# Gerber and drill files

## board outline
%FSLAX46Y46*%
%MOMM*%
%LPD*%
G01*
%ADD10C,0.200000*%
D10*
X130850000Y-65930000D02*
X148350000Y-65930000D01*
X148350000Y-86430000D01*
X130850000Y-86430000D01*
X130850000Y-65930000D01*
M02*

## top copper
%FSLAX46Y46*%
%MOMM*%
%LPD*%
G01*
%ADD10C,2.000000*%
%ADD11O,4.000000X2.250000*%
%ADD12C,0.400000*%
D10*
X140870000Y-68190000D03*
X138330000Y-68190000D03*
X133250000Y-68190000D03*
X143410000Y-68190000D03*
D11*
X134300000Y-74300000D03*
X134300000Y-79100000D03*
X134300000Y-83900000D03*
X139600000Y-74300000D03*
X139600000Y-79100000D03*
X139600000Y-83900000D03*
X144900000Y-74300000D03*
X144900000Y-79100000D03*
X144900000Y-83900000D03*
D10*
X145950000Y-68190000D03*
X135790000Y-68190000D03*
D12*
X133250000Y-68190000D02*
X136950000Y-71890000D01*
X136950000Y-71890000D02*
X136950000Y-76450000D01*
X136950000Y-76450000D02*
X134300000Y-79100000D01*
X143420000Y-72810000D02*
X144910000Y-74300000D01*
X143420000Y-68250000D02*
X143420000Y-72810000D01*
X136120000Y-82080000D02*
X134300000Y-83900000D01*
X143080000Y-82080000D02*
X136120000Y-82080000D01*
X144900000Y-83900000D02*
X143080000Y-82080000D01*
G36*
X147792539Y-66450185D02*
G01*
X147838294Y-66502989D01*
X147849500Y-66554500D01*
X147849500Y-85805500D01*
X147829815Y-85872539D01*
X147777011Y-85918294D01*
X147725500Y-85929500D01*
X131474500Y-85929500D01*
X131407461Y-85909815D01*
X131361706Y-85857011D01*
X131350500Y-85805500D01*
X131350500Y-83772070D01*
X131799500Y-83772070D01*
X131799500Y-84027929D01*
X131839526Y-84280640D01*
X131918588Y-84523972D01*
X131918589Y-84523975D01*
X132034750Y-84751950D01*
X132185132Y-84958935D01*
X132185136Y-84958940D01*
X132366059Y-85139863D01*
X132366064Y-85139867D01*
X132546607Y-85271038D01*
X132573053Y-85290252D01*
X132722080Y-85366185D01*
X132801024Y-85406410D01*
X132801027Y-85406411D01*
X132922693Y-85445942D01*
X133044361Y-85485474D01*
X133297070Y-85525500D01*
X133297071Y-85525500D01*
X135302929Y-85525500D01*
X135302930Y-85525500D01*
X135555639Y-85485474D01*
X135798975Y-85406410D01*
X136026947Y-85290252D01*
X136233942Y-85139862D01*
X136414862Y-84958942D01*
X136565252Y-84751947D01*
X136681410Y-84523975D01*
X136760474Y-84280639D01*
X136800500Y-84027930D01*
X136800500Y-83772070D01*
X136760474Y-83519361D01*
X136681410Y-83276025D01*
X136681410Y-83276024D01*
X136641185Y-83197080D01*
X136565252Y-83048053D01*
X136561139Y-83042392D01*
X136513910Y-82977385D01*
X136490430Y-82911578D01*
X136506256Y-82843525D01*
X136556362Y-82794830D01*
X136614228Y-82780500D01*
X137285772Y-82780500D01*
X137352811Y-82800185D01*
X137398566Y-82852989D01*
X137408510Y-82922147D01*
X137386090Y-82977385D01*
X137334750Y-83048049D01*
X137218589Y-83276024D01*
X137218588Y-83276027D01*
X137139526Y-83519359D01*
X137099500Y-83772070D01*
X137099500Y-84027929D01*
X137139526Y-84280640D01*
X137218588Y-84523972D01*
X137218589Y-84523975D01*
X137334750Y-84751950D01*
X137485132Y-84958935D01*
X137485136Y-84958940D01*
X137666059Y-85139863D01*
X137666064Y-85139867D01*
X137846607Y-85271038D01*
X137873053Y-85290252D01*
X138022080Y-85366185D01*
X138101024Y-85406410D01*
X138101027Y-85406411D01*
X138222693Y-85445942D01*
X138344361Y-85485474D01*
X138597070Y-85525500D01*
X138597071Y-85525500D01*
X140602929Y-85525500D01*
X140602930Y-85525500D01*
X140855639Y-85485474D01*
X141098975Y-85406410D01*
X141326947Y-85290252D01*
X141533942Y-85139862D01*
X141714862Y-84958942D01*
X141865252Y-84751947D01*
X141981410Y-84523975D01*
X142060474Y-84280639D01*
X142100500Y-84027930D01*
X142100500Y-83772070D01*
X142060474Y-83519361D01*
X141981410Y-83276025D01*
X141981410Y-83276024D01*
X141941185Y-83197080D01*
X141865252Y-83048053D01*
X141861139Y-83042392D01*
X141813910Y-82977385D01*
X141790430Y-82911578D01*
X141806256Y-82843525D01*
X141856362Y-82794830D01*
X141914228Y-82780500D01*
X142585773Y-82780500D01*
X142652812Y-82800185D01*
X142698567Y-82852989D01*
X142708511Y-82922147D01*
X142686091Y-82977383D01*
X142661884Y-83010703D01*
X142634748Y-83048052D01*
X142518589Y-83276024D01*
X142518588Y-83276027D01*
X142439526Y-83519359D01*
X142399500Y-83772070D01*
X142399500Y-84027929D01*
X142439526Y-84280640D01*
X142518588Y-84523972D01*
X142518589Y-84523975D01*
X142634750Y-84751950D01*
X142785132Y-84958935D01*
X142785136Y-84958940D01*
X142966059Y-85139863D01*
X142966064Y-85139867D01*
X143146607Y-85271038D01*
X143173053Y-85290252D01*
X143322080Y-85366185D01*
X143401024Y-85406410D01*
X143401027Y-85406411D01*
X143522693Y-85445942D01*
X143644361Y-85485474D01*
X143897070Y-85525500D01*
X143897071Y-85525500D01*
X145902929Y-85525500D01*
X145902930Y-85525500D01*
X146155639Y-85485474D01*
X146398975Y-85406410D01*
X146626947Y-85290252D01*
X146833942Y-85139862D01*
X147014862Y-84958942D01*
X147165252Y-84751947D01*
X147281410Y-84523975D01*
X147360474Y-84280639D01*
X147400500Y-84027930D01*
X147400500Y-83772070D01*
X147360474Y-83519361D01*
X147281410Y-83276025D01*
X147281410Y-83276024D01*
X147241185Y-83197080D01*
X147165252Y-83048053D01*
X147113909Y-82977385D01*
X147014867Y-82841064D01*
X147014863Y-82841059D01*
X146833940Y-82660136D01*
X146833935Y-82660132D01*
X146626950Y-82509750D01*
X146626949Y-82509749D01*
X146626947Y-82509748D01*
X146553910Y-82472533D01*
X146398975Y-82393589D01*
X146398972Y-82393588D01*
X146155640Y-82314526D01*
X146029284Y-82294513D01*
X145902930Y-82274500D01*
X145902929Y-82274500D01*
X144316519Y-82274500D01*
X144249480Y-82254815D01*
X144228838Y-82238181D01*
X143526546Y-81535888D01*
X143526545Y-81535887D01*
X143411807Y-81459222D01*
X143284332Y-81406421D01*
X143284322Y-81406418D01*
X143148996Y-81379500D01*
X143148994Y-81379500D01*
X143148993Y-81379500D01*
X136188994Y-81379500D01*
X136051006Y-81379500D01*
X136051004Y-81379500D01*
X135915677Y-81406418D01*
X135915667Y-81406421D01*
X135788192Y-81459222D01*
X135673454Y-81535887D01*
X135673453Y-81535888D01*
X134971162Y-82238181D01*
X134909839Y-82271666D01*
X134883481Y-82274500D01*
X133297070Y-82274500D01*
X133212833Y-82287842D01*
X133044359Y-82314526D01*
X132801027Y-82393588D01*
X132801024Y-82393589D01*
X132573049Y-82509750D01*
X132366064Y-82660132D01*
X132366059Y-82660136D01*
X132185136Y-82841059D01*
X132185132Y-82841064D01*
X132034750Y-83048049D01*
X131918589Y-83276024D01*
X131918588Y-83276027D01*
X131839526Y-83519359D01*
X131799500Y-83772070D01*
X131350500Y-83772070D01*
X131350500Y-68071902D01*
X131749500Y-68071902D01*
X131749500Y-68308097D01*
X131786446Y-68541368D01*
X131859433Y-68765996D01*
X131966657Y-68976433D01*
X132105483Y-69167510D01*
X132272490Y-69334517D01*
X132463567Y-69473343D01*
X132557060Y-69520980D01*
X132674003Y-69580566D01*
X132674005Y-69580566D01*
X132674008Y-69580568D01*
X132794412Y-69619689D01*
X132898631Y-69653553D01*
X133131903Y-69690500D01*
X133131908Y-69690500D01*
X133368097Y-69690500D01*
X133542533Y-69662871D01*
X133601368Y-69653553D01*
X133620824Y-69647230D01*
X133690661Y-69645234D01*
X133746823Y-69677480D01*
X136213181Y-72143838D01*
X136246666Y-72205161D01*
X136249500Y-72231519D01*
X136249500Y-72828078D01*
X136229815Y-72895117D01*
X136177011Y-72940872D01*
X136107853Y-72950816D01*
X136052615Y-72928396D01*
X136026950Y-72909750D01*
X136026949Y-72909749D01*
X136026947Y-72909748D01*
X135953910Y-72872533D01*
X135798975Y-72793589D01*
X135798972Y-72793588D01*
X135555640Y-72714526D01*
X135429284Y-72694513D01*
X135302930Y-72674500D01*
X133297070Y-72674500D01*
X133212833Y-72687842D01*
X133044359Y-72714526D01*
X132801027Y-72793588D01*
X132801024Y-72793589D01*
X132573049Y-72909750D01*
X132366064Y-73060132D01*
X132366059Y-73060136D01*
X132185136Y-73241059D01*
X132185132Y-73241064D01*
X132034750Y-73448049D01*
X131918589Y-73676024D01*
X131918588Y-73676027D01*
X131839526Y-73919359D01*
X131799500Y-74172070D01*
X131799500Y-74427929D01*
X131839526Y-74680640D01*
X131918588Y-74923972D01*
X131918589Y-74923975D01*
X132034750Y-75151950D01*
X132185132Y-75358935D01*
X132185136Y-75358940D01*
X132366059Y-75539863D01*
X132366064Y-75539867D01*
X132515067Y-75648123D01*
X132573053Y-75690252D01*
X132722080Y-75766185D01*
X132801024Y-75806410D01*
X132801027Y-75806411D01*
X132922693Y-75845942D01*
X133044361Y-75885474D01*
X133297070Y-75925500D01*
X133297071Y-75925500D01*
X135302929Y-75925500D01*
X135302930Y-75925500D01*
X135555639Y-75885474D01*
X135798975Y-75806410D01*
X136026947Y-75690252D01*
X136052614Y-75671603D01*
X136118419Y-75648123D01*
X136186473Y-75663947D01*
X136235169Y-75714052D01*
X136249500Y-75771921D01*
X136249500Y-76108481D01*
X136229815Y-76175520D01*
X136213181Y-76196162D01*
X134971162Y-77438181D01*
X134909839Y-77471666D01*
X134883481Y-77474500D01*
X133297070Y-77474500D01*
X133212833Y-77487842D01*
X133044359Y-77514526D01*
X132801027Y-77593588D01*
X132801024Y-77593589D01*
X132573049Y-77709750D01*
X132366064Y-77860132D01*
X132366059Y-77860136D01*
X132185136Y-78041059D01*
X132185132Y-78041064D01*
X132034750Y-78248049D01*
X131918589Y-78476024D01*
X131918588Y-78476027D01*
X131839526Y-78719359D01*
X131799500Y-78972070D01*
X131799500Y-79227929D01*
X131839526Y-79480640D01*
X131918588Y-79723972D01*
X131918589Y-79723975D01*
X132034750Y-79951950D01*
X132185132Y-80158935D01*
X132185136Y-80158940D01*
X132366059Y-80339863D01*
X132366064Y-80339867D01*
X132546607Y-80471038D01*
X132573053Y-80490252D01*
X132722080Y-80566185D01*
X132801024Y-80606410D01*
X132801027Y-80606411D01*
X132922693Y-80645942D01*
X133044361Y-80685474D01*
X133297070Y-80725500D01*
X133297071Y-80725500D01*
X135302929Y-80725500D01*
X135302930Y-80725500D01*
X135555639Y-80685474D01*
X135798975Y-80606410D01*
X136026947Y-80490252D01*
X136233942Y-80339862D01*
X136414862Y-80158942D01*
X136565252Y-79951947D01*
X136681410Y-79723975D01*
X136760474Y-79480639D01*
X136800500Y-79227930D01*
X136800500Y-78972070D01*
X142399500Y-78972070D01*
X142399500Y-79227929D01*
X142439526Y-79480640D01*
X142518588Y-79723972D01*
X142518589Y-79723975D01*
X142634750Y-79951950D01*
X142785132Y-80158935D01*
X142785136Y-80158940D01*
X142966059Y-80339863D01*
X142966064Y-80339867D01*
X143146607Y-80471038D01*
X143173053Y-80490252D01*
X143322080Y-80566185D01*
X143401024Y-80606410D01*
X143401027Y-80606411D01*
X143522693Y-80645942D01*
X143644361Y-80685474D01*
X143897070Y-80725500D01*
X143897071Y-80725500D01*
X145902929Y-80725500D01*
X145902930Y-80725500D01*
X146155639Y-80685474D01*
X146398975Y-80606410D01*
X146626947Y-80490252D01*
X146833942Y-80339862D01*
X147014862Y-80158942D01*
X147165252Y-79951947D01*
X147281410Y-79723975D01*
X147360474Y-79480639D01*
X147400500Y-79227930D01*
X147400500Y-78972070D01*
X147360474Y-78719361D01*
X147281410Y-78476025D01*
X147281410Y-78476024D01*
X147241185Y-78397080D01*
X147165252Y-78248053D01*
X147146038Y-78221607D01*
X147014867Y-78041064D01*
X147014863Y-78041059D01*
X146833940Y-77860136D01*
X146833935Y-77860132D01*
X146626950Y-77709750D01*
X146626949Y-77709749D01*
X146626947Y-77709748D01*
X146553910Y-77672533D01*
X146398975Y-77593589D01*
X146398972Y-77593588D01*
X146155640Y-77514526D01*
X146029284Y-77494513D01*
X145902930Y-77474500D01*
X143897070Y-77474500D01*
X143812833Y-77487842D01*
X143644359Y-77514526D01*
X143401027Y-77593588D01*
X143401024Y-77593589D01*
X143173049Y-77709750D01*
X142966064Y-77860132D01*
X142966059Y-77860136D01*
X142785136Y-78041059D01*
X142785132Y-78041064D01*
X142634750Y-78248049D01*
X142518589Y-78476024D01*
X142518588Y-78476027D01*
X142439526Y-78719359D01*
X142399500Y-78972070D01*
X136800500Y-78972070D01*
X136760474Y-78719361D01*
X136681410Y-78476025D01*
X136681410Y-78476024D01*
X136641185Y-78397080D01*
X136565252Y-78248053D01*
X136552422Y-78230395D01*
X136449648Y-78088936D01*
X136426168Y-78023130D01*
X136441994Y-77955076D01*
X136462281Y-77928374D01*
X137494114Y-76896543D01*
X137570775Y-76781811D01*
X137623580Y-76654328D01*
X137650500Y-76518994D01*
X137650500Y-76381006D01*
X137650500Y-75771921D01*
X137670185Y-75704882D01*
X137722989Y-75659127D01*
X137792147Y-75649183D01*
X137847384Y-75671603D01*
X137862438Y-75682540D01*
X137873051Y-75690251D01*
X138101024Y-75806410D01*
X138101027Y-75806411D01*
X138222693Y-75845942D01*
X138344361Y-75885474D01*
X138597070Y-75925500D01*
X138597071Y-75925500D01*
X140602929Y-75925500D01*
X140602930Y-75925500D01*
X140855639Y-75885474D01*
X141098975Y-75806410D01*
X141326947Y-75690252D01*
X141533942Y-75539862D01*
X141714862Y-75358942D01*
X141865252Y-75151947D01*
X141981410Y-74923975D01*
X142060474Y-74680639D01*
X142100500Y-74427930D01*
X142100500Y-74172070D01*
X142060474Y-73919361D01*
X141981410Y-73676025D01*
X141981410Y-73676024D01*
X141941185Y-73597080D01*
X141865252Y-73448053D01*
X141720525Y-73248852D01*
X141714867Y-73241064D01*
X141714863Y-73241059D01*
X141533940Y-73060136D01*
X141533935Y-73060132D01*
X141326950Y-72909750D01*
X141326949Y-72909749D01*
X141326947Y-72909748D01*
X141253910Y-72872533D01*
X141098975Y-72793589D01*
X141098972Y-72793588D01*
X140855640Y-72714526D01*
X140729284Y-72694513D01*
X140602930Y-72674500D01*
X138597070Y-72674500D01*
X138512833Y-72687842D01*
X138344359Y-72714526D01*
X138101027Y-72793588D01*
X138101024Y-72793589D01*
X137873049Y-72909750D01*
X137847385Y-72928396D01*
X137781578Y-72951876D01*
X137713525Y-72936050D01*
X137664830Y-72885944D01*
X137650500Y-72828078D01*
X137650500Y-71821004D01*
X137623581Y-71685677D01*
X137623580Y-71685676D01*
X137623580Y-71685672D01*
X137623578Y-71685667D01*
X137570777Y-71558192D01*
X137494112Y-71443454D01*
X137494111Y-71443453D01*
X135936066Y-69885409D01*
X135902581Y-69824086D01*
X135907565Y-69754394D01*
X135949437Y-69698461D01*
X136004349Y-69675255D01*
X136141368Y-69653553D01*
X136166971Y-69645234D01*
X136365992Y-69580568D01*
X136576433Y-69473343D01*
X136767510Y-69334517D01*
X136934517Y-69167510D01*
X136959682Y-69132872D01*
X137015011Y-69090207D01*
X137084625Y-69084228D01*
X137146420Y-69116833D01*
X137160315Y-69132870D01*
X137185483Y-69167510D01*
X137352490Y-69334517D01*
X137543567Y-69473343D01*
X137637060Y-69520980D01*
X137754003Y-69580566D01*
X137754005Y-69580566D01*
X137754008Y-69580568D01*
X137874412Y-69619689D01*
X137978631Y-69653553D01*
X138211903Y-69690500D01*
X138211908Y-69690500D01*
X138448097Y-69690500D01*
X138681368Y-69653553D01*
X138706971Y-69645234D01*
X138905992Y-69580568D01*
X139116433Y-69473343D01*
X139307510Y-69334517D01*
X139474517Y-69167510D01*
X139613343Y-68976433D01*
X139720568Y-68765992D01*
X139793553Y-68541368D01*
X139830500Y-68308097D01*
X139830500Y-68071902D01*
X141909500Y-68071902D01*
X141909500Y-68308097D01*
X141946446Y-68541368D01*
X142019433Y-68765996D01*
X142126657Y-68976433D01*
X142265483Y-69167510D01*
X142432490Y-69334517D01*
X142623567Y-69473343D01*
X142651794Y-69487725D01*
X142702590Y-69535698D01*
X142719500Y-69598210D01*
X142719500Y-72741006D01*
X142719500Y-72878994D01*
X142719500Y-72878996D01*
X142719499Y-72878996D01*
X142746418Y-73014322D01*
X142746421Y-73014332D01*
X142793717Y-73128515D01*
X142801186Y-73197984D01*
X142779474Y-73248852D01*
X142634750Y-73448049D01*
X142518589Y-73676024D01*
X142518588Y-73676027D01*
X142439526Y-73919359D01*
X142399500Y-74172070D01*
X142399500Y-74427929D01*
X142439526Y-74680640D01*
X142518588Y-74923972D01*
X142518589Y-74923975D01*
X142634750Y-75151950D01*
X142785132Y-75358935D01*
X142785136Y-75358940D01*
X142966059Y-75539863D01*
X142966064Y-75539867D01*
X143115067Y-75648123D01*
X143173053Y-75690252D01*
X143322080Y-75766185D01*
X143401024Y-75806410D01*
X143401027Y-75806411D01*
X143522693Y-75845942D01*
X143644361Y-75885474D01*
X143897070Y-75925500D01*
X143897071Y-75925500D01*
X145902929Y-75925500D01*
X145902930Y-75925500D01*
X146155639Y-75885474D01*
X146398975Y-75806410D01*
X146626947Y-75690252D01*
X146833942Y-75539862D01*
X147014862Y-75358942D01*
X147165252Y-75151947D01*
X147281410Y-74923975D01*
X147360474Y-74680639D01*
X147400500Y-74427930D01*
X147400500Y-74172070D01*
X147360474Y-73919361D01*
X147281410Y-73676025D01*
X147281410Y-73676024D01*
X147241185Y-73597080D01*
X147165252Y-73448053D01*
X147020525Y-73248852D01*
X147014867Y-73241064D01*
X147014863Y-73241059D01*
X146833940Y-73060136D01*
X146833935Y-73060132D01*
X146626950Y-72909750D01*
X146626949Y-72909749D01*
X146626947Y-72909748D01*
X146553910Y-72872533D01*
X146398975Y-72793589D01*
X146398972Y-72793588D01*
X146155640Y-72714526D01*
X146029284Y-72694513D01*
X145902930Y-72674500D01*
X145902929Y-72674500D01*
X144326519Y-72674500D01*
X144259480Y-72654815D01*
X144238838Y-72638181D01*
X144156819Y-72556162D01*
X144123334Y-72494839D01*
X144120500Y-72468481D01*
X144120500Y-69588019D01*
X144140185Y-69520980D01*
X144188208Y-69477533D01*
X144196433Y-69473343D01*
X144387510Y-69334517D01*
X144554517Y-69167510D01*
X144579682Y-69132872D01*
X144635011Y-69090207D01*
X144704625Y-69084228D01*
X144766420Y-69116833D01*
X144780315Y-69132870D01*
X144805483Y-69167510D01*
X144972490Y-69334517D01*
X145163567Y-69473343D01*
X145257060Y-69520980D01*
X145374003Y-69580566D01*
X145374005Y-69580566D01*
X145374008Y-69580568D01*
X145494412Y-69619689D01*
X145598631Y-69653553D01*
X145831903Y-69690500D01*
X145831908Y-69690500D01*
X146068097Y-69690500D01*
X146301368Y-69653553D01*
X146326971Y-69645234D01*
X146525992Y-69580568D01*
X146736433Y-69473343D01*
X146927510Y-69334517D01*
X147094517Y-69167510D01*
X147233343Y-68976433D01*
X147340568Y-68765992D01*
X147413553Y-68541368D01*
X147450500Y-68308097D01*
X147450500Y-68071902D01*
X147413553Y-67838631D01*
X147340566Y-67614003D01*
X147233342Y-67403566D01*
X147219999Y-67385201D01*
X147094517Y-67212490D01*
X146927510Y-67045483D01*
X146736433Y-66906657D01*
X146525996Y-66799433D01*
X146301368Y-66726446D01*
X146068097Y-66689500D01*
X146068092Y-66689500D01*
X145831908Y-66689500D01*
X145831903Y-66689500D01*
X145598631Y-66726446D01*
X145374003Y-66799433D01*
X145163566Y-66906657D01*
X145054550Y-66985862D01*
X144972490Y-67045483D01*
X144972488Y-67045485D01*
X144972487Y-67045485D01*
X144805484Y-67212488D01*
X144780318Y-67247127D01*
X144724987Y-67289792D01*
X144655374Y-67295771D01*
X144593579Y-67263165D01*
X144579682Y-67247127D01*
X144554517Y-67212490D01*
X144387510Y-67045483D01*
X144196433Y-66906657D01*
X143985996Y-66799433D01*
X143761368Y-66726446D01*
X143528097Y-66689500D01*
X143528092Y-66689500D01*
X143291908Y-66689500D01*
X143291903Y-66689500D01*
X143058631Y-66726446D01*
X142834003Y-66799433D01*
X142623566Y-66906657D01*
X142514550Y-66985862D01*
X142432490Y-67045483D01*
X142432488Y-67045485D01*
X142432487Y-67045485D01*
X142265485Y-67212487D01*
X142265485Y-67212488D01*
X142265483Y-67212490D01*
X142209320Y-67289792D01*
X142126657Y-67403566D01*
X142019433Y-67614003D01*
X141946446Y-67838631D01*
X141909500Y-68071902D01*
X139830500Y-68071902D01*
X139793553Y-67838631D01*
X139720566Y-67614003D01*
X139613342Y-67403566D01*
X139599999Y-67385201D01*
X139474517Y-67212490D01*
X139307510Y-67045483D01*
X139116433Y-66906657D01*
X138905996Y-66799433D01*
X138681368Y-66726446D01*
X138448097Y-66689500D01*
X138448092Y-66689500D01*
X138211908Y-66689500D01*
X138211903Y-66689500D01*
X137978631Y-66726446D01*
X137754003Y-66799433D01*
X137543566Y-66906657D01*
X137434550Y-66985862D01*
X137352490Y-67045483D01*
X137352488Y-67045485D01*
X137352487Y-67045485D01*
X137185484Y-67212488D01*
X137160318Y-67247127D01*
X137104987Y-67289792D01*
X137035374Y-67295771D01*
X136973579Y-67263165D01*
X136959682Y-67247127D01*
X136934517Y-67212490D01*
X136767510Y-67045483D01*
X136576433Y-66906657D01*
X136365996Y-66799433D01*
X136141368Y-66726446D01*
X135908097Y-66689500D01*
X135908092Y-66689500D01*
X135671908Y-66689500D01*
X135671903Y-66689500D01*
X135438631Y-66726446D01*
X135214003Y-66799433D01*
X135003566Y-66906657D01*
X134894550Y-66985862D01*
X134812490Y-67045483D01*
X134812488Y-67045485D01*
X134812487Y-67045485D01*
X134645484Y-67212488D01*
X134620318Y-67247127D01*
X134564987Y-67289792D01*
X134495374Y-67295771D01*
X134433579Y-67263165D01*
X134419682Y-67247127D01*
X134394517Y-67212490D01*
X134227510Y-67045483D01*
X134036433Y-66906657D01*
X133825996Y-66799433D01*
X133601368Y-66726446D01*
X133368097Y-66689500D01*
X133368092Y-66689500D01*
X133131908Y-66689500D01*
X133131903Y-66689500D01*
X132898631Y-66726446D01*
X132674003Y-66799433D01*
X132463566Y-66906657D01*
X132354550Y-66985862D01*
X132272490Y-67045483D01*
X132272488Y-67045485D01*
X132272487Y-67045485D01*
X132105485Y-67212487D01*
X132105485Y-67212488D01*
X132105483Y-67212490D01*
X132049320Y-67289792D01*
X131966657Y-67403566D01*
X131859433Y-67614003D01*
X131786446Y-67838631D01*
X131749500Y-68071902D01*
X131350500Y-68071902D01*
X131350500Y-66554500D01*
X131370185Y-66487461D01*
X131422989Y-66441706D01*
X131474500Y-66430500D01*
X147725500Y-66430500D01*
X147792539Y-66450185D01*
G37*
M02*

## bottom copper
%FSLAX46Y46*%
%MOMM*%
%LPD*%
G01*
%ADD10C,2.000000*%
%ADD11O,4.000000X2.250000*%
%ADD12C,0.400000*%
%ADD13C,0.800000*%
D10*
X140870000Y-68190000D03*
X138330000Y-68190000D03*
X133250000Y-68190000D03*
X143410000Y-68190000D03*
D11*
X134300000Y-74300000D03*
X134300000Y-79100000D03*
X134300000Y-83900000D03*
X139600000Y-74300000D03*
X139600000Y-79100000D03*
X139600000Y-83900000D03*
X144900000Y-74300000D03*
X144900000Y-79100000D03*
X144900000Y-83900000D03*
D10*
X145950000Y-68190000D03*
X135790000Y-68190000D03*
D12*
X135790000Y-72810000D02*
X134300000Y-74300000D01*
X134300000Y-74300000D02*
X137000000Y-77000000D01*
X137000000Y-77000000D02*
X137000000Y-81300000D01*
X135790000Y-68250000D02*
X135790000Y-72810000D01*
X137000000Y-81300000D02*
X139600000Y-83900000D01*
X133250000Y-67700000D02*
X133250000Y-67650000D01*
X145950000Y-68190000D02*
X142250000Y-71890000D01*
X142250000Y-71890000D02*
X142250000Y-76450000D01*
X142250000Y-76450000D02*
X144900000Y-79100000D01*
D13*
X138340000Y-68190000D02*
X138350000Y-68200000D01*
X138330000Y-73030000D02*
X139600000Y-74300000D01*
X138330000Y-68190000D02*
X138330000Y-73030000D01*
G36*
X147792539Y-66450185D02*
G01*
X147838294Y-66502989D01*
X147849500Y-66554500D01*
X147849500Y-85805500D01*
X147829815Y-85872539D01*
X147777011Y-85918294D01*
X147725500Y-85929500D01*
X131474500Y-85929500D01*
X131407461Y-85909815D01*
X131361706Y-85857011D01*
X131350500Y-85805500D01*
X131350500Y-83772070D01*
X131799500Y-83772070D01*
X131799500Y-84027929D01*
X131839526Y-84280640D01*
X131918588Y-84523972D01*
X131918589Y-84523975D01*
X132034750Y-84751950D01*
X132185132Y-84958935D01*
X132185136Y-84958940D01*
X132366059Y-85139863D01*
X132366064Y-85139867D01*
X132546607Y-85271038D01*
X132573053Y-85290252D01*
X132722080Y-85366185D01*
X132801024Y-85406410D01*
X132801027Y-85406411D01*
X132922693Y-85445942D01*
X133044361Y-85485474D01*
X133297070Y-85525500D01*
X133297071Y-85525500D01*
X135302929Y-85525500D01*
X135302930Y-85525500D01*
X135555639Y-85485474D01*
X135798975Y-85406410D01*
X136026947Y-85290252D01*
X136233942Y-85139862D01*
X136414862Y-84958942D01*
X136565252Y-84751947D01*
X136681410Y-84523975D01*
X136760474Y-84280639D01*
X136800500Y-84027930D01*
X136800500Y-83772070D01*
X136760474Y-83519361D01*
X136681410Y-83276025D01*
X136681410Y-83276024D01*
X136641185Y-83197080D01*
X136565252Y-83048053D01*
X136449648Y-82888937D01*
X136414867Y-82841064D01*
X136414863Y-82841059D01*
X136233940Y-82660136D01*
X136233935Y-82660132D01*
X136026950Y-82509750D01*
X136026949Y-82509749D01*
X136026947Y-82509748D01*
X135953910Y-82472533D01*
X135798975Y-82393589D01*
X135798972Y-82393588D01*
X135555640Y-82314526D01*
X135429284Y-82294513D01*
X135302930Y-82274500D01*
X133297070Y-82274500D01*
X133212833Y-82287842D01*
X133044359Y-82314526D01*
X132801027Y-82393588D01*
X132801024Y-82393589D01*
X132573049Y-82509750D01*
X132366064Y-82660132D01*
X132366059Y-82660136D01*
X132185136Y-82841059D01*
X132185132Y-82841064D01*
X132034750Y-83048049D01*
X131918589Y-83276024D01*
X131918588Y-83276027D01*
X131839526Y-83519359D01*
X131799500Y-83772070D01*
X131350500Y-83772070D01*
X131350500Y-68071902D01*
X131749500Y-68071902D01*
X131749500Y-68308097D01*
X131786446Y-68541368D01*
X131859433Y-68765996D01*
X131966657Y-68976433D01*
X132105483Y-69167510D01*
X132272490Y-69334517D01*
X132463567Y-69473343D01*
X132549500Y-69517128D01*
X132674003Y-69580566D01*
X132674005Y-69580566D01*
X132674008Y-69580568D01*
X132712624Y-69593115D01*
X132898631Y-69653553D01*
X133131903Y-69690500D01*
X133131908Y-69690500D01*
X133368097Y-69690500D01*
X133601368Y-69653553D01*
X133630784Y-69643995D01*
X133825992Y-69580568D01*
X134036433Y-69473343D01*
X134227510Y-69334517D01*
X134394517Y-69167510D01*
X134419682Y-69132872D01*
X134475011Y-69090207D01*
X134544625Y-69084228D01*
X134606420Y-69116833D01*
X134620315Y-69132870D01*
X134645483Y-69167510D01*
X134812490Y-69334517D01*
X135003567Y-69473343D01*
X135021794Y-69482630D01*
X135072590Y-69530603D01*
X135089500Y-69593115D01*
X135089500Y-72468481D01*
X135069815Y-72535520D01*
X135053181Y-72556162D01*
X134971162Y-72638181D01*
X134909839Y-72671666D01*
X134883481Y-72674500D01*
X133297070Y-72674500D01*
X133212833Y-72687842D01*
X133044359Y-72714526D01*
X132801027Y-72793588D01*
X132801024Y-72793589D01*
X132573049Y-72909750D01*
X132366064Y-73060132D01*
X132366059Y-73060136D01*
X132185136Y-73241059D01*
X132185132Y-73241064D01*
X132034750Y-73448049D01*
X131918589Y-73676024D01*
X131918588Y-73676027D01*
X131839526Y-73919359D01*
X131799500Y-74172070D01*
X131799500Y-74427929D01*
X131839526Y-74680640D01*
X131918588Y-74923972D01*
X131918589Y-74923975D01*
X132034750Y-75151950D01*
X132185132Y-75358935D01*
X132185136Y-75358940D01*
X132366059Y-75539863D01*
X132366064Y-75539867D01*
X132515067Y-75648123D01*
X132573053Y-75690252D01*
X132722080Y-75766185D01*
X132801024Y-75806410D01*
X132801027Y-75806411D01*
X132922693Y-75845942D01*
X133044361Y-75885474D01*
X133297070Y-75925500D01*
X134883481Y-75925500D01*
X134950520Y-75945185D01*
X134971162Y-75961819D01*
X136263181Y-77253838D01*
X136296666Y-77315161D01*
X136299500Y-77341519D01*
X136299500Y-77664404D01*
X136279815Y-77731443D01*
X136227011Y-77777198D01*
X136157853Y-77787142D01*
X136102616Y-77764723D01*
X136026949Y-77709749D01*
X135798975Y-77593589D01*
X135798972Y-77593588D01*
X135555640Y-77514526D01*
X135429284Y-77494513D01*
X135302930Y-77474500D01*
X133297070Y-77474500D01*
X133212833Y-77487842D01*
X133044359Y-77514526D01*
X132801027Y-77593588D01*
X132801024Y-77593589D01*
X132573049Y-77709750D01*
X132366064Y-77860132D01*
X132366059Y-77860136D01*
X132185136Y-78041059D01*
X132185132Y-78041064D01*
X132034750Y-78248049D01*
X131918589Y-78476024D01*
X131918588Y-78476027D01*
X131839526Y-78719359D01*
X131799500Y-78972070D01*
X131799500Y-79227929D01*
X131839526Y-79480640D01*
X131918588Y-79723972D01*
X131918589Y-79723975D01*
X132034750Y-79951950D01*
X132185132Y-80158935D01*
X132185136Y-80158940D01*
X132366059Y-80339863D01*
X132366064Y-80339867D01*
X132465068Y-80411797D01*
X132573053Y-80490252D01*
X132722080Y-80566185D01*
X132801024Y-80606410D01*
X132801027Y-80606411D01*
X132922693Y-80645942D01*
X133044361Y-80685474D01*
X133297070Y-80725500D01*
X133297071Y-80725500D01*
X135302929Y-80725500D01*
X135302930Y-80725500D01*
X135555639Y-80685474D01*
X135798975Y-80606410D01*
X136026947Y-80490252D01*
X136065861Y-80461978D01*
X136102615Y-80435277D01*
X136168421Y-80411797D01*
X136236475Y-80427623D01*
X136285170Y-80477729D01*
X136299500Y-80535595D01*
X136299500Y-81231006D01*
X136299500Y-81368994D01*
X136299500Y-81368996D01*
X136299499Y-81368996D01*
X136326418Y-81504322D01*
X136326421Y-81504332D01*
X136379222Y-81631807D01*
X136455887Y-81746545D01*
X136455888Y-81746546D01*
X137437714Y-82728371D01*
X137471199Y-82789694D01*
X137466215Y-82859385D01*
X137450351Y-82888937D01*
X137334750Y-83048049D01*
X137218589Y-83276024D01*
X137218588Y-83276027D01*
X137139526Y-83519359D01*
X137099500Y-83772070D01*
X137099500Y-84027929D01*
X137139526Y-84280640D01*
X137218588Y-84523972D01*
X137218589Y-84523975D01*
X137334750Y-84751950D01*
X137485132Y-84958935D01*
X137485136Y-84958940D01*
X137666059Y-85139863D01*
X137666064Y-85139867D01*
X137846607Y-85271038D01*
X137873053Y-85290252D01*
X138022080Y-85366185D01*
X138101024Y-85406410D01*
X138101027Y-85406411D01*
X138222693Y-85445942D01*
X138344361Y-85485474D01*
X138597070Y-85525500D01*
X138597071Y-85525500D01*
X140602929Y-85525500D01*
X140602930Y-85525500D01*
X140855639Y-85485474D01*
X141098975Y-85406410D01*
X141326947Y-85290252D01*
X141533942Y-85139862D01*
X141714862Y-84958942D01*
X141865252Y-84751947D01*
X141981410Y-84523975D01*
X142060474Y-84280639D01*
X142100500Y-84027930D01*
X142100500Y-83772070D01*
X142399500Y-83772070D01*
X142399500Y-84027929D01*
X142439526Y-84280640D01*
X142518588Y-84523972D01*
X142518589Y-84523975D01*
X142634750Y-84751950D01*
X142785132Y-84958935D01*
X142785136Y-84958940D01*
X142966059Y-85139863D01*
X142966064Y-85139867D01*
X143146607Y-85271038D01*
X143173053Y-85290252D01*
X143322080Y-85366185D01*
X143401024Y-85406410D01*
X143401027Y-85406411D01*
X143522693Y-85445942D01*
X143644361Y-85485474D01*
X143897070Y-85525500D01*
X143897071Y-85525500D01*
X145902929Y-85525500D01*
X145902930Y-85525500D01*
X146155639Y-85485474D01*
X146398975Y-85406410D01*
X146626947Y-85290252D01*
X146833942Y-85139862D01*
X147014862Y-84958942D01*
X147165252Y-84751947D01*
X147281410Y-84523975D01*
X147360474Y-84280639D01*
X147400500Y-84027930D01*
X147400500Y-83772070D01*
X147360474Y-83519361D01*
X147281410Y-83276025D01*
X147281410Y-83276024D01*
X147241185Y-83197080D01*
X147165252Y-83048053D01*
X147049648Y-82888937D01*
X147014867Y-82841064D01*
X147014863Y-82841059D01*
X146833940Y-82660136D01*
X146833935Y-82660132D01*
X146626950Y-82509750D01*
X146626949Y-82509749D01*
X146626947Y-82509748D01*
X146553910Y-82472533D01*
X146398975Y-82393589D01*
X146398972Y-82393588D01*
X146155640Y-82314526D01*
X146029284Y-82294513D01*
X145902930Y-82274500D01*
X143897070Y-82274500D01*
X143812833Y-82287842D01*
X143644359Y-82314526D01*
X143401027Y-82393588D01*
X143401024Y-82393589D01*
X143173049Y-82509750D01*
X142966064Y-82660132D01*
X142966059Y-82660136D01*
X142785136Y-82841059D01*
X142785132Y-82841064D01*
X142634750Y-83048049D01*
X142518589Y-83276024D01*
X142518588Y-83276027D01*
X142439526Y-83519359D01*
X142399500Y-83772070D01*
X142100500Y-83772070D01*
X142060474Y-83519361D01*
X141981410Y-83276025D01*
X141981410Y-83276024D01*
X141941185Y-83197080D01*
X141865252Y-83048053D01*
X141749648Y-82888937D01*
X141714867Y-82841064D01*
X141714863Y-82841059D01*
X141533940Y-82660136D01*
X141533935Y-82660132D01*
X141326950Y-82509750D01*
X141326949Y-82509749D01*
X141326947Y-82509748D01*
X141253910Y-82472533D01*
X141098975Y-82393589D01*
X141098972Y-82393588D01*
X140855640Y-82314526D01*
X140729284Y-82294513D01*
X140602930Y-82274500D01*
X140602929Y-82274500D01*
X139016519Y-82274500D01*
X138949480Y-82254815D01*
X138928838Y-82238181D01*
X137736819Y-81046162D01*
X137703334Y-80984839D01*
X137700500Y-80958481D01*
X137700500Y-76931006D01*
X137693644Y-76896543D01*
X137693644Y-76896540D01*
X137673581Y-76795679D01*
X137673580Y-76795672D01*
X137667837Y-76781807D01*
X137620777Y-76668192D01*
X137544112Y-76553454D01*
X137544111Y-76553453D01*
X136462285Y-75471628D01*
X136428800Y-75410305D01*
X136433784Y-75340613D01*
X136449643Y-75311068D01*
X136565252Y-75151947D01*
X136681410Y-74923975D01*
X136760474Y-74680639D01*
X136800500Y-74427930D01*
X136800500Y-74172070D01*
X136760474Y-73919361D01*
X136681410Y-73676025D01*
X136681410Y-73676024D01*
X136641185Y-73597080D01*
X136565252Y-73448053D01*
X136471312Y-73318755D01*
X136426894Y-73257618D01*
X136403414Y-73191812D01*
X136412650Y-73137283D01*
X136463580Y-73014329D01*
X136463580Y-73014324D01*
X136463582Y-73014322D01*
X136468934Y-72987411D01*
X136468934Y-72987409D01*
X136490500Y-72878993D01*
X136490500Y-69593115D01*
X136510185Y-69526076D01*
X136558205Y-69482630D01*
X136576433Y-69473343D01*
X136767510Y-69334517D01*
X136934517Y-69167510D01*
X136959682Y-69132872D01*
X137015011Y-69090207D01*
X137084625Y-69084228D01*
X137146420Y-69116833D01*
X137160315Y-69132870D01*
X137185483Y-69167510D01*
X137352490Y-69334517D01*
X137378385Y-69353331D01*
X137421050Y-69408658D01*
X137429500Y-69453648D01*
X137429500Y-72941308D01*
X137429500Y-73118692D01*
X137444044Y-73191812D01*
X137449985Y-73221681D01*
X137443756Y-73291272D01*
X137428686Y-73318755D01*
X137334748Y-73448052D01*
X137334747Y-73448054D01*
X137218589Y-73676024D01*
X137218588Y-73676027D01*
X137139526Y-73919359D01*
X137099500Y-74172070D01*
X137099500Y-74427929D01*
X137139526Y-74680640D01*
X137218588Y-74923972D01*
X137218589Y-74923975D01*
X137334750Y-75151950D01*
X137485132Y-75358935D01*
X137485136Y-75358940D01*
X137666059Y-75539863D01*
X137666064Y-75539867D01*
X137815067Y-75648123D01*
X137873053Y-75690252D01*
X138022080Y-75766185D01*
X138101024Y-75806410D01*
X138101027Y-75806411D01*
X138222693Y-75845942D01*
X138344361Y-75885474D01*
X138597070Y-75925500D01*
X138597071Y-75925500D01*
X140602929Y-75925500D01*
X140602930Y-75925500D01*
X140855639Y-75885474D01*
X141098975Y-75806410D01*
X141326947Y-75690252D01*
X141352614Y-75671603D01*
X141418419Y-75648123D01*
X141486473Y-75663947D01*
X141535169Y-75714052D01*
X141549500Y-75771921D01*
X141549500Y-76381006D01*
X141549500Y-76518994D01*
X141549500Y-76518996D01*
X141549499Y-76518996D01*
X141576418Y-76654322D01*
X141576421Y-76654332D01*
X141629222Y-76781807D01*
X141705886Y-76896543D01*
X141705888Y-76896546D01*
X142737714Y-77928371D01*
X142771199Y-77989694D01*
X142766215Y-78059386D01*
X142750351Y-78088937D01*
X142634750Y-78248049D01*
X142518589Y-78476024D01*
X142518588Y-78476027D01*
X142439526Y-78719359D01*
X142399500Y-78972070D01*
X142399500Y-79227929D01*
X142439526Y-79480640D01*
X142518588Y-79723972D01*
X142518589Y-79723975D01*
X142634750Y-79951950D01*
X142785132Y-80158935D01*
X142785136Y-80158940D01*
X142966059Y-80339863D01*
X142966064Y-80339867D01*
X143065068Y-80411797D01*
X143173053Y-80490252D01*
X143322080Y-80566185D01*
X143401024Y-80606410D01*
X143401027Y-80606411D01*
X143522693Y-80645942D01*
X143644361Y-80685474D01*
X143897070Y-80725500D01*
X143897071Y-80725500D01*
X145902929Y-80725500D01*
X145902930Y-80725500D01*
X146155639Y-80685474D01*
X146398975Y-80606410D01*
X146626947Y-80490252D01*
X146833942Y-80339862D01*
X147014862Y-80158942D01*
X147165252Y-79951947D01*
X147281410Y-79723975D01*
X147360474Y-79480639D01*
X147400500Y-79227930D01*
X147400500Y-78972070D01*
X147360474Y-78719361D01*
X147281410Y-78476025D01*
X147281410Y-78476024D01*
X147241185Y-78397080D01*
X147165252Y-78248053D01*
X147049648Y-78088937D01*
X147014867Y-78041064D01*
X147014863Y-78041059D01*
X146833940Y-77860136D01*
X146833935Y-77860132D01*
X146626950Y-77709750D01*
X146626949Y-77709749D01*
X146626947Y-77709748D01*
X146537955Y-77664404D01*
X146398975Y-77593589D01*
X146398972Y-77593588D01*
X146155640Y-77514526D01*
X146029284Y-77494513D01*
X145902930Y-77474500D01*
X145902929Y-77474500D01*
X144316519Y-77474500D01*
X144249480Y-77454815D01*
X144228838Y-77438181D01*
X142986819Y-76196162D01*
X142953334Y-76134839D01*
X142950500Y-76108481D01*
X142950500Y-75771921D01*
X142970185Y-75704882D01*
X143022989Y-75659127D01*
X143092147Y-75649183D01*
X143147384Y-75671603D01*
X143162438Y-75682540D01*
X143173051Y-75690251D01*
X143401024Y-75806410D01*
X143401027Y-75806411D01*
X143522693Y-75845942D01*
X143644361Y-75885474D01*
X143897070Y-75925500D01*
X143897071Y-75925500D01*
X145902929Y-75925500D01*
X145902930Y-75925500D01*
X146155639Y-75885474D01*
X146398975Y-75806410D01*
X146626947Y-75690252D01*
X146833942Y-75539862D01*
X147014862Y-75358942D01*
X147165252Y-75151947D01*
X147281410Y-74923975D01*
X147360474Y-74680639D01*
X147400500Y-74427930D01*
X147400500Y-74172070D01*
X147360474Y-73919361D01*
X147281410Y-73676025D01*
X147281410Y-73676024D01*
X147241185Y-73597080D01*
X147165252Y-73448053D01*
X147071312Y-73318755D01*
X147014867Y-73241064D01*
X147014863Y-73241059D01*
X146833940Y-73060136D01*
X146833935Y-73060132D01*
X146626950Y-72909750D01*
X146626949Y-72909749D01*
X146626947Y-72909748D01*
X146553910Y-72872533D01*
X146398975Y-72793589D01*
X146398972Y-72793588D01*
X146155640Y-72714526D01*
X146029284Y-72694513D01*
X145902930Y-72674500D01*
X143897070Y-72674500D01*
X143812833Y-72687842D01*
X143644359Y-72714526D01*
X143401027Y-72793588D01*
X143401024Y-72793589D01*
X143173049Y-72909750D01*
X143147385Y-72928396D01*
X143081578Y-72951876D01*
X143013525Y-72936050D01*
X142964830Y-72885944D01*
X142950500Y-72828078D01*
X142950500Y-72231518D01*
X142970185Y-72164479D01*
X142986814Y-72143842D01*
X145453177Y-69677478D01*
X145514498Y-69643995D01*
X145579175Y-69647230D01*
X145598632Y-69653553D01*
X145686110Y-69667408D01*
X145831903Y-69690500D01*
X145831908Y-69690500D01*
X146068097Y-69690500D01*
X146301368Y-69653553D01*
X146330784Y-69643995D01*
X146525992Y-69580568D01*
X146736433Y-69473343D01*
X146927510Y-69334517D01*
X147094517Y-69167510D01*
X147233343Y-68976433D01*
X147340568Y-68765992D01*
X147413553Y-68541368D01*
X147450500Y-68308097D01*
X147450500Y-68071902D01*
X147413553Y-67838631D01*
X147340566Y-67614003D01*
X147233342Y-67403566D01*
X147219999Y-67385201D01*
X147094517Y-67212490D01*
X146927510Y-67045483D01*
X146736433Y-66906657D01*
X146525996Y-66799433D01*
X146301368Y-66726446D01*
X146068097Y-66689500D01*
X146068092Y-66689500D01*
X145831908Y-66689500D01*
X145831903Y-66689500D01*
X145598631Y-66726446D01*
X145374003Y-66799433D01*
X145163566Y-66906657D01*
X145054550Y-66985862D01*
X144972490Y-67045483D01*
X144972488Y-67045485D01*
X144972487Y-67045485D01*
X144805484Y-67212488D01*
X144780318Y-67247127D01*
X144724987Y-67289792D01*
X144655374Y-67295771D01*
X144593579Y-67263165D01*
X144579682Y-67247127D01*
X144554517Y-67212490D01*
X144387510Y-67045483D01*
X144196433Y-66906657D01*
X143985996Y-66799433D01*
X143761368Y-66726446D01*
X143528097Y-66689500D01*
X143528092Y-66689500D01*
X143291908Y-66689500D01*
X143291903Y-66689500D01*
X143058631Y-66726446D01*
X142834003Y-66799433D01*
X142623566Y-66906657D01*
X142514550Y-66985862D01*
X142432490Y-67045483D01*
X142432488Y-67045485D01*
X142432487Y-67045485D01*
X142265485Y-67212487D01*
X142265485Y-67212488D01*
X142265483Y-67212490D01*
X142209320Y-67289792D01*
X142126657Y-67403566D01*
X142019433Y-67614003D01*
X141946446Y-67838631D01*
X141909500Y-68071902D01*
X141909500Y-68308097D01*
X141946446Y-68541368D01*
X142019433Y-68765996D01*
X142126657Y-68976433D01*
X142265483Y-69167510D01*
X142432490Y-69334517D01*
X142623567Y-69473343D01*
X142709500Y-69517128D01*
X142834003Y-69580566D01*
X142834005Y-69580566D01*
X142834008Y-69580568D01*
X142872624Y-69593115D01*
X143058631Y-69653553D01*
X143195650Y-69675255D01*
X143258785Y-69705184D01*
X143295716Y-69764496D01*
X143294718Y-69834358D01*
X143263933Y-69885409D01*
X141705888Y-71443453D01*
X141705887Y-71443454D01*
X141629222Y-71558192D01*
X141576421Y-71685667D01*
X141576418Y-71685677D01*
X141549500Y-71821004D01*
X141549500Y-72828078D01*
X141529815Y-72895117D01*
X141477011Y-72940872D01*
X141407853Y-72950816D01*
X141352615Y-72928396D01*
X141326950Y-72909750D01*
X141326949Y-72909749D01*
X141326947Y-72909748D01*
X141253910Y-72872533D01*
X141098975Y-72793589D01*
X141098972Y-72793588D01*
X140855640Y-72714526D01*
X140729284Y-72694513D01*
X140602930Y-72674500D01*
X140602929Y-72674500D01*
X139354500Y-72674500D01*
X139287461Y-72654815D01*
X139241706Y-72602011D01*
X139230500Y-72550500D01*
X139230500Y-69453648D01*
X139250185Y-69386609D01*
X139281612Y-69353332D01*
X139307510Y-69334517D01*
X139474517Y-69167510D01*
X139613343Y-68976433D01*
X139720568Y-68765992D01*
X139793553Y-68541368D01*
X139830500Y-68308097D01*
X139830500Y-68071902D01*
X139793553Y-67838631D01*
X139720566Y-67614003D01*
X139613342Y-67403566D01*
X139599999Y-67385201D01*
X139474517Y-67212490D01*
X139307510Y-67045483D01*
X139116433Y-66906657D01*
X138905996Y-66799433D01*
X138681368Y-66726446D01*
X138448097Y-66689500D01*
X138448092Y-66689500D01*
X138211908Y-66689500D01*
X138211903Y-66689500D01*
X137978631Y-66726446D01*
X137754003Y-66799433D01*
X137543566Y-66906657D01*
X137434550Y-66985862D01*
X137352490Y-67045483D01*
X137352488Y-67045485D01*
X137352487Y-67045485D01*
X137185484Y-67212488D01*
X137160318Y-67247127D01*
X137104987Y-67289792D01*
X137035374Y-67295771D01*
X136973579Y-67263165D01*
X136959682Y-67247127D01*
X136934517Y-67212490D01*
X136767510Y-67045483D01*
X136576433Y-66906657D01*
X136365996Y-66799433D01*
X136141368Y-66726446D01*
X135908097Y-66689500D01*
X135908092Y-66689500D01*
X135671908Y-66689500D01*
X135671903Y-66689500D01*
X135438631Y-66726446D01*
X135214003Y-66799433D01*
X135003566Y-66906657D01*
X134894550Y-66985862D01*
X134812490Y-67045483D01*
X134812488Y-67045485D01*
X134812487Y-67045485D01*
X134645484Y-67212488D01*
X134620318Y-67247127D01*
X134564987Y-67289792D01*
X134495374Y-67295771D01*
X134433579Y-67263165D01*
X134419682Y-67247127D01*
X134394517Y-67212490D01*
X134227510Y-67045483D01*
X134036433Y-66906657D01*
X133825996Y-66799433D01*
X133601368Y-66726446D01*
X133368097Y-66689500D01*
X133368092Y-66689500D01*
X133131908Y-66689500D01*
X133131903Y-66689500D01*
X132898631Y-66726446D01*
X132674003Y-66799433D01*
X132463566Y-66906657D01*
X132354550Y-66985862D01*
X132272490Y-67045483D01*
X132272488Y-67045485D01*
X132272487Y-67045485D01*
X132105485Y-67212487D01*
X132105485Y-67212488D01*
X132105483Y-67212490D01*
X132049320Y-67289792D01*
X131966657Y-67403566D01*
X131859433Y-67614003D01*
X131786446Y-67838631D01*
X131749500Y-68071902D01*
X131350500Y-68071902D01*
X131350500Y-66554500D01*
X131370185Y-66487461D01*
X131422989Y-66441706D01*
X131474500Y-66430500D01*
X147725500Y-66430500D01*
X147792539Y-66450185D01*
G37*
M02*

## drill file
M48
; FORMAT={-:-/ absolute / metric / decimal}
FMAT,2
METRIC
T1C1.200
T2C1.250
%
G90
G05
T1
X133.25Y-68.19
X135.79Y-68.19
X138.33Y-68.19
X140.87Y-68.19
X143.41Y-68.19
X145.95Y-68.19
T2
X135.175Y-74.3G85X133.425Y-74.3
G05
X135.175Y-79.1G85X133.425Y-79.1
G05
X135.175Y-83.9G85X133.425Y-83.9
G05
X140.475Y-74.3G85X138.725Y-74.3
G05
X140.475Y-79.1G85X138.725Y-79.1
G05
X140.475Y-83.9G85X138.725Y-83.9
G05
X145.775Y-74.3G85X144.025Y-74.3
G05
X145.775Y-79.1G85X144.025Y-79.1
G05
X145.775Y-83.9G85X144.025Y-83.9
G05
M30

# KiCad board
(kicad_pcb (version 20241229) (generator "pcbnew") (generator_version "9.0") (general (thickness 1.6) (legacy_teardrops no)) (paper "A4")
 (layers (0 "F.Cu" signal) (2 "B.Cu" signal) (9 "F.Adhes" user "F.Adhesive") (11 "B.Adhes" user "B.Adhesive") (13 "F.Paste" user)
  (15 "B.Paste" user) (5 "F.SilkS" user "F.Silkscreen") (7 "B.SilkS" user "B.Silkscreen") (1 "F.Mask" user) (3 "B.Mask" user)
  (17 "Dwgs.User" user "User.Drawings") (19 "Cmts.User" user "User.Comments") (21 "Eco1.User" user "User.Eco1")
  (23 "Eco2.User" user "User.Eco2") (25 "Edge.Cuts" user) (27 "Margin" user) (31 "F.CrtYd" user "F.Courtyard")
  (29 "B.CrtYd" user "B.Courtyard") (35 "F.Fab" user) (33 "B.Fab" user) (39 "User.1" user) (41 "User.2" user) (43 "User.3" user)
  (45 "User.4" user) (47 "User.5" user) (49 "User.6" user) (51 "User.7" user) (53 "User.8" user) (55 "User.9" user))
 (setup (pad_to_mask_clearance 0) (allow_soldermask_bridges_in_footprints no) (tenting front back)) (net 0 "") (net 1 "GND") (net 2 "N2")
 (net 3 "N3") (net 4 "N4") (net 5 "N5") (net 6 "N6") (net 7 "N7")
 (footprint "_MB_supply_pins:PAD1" (layer "F.Cu") (at 140.87 68.19)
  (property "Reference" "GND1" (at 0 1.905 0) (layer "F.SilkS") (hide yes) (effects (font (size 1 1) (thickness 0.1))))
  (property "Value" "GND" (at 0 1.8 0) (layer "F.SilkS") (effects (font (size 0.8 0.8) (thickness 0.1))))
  (pad "1" thru_hole circle (at 0 0) (size 2 2) (drill 1.2) (layers "*.Cu" "*.Mask") (remove_unused_layers no) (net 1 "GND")))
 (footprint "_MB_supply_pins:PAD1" (layer "F.Cu") (at 138.33 68.19)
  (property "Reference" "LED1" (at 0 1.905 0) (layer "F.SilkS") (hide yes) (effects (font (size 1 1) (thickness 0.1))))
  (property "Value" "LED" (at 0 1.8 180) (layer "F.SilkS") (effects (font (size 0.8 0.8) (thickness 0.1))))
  (pad "1" thru_hole circle (at 0 0) (size 2 2) (drill 1.2) (layers "*.Cu" "*.Mask") (remove_unused_layers no) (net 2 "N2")))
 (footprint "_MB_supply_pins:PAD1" (layer "F.Cu") (at 133.25 68.19)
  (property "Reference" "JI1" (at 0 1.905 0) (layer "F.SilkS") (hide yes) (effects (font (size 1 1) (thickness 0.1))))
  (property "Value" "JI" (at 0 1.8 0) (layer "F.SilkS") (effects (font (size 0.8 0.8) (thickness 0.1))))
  (pad "1" thru_hole circle (at 0 0) (size 2 2) (drill 1.2) (layers "*.Cu" "*.Mask") (remove_unused_layers no) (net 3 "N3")))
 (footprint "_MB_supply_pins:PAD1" (layer "F.Cu") (at 143.41 68.19)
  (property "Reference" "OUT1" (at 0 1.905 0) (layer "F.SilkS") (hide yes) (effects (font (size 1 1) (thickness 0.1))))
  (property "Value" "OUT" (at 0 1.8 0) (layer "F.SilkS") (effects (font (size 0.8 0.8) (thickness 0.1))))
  (pad "1" thru_hole circle (at 0 0) (size 2 2) (drill 1.2) (layers "*.Cu" "*.Mask") (remove_unused_layers no) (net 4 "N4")))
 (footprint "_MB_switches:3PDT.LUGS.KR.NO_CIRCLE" (layer "F.Cu") (at 139.6 79.1)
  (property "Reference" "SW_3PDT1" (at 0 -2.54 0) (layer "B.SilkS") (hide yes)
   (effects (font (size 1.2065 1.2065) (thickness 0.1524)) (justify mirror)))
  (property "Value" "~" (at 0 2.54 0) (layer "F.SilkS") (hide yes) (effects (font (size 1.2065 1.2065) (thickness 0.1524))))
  (pad "1" thru_hole oval (at -5.3 -4.8 180) (size 4 2.25) (drill oval 3 1.25) (layers "*.Cu" "*.Mask") (remove_unused_layers no)
   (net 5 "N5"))
  (pad "2" thru_hole oval (at -5.3 0 180) (size 4 2.25) (drill oval 3 1.25) (layers "*.Cu" "*.Mask") (remove_unused_layers no) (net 3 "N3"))
  (pad "3" thru_hole oval (at -5.3 4.8 180) (size 4 2.25) (drill oval 3 1.25) (layers "*.Cu" "*.Mask") (remove_unused_layers no)
   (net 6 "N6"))
  (pad "4" thru_hole oval (at 0 -4.8 180) (size 4 2.25) (drill oval 3 1.25) (layers "*.Cu" "*.Mask") (remove_unused_layers no) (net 2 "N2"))
  (pad "5" thru_hole oval (at 0 0 180) (size 4 2.25) (drill oval 3 1.25) (layers "*.Cu" "*.Mask") (remove_unused_layers no) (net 1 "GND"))
  (pad "6" thru_hole oval (at 0 4.8 180) (size 4 2.25) (drill oval 3 1.25) (layers "*.Cu" "*.Mask") (remove_unused_layers no) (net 5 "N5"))
  (pad "7" thru_hole oval (at 5.3 -4.8 180) (size 4 2.25) (drill oval 3 1.25) (layers "*.Cu" "*.Mask") (remove_unused_layers no)
   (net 4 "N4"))
  (pad "8" thru_hole oval (at 5.3 0 180) (size 4 2.25) (drill oval 3 1.25) (layers "*.Cu" "*.Mask") (remove_unused_layers no) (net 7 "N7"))
  (pad "9" thru_hole oval (at 5.3 4.8 180) (size 4 2.25) (drill oval 3 1.25) (layers "*.Cu" "*.Mask") (remove_unused_layers no) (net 6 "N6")))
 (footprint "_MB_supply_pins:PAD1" (layer "F.Cu") (at 145.95 68.19)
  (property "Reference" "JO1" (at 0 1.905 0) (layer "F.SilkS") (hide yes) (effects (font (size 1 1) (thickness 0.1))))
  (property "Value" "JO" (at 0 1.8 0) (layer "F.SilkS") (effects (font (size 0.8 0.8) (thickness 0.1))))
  (pad "1" thru_hole circle (at 0 0) (size 2 2) (drill 1.2) (layers "*.Cu" "*.Mask") (remove_unused_layers no) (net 7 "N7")))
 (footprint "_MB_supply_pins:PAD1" (layer "F.Cu") (at 135.79 68.19)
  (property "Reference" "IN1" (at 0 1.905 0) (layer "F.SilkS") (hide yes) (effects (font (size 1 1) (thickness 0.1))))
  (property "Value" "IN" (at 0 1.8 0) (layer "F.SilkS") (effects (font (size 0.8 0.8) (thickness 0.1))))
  (pad "1" thru_hole circle (at 0 0) (size 2 2) (drill 1.2) (layers "*.Cu" "*.Mask") (remove_unused_layers no) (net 5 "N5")))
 (gr_rect (start 130.85 65.93) (end 148.35 86.43) (stroke (width 0.2) (type default)) (fill no) (layer "Edge.Cuts"))
 (segment (start 135.79 72.81) (end 134.3 74.3) (width 0.4) (layer "B.Cu") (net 5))
 (segment (start 134.3 74.3) (end 137 77) (width 0.4) (layer "B.Cu") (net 5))
 (segment (start 137 77) (end 137 81.3) (width 0.4) (layer "B.Cu") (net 5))
 (segment (start 135.79 68.25) (end 135.79 72.81) (width 0.4) (layer "B.Cu") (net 5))
 (segment (start 137 81.3) (end 139.6 83.9) (width 0.4) (layer "B.Cu") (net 5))
 (segment (start 133.25 68.19) (end 136.95 71.89) (width 0.4) (layer "F.Cu") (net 3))
 (segment (start 136.95 71.89) (end 136.95 76.45) (width 0.4) (layer "F.Cu") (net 3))
 (segment (start 136.95 76.45) (end 134.3 79.1) (width 0.4) (layer "F.Cu") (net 3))
 (segment (start 133.25 67.7) (end 133.25 67.65) (width 0.4) (layer "B.Cu") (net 3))
 (segment (start 145.95 68.19) (end 142.25 71.89) (width 0.4) (layer "B.Cu") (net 7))
 (segment (start 142.25 71.89) (end 142.25 76.45) (width 0.4) (layer "B.Cu") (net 7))
 (segment (start 142.25 76.45) (end 144.9 79.1) (width 0.4) (layer "B.Cu") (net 7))
 (segment (start 138.34 68.19) (end 138.35 68.2) (width 0.8) (layer "B.Cu") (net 2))
 (segment (start 138.33 73.03) (end 139.6 74.3) (width 0.8) (layer "B.Cu") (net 2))
 (segment (start 138.33 68.19) (end 138.33 73.03) (width 0.8) (layer "B.Cu") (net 2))
 (segment (start 143.42 72.81) (end 144.91 74.3) (width 0.4) (layer "F.Cu") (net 4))
 (segment (start 143.42 68.25) (end 143.42 72.81) (width 0.4) (layer "F.Cu") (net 4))
 (segment (start 136.12 82.08) (end 134.3 83.9) (width 0.4) (layer "F.Cu") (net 6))
 (segment (start 143.08 82.08) (end 136.12 82.08) (width 0.4) (layer "F.Cu") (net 6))
 (segment (start 144.9 83.9) (end 143.08 82.08) (width 0.4) (layer "F.Cu") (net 6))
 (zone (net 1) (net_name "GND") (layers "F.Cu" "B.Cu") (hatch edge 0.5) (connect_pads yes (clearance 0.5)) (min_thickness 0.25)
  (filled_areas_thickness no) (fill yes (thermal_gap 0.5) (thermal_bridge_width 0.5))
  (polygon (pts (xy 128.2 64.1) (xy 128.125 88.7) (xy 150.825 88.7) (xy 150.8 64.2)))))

